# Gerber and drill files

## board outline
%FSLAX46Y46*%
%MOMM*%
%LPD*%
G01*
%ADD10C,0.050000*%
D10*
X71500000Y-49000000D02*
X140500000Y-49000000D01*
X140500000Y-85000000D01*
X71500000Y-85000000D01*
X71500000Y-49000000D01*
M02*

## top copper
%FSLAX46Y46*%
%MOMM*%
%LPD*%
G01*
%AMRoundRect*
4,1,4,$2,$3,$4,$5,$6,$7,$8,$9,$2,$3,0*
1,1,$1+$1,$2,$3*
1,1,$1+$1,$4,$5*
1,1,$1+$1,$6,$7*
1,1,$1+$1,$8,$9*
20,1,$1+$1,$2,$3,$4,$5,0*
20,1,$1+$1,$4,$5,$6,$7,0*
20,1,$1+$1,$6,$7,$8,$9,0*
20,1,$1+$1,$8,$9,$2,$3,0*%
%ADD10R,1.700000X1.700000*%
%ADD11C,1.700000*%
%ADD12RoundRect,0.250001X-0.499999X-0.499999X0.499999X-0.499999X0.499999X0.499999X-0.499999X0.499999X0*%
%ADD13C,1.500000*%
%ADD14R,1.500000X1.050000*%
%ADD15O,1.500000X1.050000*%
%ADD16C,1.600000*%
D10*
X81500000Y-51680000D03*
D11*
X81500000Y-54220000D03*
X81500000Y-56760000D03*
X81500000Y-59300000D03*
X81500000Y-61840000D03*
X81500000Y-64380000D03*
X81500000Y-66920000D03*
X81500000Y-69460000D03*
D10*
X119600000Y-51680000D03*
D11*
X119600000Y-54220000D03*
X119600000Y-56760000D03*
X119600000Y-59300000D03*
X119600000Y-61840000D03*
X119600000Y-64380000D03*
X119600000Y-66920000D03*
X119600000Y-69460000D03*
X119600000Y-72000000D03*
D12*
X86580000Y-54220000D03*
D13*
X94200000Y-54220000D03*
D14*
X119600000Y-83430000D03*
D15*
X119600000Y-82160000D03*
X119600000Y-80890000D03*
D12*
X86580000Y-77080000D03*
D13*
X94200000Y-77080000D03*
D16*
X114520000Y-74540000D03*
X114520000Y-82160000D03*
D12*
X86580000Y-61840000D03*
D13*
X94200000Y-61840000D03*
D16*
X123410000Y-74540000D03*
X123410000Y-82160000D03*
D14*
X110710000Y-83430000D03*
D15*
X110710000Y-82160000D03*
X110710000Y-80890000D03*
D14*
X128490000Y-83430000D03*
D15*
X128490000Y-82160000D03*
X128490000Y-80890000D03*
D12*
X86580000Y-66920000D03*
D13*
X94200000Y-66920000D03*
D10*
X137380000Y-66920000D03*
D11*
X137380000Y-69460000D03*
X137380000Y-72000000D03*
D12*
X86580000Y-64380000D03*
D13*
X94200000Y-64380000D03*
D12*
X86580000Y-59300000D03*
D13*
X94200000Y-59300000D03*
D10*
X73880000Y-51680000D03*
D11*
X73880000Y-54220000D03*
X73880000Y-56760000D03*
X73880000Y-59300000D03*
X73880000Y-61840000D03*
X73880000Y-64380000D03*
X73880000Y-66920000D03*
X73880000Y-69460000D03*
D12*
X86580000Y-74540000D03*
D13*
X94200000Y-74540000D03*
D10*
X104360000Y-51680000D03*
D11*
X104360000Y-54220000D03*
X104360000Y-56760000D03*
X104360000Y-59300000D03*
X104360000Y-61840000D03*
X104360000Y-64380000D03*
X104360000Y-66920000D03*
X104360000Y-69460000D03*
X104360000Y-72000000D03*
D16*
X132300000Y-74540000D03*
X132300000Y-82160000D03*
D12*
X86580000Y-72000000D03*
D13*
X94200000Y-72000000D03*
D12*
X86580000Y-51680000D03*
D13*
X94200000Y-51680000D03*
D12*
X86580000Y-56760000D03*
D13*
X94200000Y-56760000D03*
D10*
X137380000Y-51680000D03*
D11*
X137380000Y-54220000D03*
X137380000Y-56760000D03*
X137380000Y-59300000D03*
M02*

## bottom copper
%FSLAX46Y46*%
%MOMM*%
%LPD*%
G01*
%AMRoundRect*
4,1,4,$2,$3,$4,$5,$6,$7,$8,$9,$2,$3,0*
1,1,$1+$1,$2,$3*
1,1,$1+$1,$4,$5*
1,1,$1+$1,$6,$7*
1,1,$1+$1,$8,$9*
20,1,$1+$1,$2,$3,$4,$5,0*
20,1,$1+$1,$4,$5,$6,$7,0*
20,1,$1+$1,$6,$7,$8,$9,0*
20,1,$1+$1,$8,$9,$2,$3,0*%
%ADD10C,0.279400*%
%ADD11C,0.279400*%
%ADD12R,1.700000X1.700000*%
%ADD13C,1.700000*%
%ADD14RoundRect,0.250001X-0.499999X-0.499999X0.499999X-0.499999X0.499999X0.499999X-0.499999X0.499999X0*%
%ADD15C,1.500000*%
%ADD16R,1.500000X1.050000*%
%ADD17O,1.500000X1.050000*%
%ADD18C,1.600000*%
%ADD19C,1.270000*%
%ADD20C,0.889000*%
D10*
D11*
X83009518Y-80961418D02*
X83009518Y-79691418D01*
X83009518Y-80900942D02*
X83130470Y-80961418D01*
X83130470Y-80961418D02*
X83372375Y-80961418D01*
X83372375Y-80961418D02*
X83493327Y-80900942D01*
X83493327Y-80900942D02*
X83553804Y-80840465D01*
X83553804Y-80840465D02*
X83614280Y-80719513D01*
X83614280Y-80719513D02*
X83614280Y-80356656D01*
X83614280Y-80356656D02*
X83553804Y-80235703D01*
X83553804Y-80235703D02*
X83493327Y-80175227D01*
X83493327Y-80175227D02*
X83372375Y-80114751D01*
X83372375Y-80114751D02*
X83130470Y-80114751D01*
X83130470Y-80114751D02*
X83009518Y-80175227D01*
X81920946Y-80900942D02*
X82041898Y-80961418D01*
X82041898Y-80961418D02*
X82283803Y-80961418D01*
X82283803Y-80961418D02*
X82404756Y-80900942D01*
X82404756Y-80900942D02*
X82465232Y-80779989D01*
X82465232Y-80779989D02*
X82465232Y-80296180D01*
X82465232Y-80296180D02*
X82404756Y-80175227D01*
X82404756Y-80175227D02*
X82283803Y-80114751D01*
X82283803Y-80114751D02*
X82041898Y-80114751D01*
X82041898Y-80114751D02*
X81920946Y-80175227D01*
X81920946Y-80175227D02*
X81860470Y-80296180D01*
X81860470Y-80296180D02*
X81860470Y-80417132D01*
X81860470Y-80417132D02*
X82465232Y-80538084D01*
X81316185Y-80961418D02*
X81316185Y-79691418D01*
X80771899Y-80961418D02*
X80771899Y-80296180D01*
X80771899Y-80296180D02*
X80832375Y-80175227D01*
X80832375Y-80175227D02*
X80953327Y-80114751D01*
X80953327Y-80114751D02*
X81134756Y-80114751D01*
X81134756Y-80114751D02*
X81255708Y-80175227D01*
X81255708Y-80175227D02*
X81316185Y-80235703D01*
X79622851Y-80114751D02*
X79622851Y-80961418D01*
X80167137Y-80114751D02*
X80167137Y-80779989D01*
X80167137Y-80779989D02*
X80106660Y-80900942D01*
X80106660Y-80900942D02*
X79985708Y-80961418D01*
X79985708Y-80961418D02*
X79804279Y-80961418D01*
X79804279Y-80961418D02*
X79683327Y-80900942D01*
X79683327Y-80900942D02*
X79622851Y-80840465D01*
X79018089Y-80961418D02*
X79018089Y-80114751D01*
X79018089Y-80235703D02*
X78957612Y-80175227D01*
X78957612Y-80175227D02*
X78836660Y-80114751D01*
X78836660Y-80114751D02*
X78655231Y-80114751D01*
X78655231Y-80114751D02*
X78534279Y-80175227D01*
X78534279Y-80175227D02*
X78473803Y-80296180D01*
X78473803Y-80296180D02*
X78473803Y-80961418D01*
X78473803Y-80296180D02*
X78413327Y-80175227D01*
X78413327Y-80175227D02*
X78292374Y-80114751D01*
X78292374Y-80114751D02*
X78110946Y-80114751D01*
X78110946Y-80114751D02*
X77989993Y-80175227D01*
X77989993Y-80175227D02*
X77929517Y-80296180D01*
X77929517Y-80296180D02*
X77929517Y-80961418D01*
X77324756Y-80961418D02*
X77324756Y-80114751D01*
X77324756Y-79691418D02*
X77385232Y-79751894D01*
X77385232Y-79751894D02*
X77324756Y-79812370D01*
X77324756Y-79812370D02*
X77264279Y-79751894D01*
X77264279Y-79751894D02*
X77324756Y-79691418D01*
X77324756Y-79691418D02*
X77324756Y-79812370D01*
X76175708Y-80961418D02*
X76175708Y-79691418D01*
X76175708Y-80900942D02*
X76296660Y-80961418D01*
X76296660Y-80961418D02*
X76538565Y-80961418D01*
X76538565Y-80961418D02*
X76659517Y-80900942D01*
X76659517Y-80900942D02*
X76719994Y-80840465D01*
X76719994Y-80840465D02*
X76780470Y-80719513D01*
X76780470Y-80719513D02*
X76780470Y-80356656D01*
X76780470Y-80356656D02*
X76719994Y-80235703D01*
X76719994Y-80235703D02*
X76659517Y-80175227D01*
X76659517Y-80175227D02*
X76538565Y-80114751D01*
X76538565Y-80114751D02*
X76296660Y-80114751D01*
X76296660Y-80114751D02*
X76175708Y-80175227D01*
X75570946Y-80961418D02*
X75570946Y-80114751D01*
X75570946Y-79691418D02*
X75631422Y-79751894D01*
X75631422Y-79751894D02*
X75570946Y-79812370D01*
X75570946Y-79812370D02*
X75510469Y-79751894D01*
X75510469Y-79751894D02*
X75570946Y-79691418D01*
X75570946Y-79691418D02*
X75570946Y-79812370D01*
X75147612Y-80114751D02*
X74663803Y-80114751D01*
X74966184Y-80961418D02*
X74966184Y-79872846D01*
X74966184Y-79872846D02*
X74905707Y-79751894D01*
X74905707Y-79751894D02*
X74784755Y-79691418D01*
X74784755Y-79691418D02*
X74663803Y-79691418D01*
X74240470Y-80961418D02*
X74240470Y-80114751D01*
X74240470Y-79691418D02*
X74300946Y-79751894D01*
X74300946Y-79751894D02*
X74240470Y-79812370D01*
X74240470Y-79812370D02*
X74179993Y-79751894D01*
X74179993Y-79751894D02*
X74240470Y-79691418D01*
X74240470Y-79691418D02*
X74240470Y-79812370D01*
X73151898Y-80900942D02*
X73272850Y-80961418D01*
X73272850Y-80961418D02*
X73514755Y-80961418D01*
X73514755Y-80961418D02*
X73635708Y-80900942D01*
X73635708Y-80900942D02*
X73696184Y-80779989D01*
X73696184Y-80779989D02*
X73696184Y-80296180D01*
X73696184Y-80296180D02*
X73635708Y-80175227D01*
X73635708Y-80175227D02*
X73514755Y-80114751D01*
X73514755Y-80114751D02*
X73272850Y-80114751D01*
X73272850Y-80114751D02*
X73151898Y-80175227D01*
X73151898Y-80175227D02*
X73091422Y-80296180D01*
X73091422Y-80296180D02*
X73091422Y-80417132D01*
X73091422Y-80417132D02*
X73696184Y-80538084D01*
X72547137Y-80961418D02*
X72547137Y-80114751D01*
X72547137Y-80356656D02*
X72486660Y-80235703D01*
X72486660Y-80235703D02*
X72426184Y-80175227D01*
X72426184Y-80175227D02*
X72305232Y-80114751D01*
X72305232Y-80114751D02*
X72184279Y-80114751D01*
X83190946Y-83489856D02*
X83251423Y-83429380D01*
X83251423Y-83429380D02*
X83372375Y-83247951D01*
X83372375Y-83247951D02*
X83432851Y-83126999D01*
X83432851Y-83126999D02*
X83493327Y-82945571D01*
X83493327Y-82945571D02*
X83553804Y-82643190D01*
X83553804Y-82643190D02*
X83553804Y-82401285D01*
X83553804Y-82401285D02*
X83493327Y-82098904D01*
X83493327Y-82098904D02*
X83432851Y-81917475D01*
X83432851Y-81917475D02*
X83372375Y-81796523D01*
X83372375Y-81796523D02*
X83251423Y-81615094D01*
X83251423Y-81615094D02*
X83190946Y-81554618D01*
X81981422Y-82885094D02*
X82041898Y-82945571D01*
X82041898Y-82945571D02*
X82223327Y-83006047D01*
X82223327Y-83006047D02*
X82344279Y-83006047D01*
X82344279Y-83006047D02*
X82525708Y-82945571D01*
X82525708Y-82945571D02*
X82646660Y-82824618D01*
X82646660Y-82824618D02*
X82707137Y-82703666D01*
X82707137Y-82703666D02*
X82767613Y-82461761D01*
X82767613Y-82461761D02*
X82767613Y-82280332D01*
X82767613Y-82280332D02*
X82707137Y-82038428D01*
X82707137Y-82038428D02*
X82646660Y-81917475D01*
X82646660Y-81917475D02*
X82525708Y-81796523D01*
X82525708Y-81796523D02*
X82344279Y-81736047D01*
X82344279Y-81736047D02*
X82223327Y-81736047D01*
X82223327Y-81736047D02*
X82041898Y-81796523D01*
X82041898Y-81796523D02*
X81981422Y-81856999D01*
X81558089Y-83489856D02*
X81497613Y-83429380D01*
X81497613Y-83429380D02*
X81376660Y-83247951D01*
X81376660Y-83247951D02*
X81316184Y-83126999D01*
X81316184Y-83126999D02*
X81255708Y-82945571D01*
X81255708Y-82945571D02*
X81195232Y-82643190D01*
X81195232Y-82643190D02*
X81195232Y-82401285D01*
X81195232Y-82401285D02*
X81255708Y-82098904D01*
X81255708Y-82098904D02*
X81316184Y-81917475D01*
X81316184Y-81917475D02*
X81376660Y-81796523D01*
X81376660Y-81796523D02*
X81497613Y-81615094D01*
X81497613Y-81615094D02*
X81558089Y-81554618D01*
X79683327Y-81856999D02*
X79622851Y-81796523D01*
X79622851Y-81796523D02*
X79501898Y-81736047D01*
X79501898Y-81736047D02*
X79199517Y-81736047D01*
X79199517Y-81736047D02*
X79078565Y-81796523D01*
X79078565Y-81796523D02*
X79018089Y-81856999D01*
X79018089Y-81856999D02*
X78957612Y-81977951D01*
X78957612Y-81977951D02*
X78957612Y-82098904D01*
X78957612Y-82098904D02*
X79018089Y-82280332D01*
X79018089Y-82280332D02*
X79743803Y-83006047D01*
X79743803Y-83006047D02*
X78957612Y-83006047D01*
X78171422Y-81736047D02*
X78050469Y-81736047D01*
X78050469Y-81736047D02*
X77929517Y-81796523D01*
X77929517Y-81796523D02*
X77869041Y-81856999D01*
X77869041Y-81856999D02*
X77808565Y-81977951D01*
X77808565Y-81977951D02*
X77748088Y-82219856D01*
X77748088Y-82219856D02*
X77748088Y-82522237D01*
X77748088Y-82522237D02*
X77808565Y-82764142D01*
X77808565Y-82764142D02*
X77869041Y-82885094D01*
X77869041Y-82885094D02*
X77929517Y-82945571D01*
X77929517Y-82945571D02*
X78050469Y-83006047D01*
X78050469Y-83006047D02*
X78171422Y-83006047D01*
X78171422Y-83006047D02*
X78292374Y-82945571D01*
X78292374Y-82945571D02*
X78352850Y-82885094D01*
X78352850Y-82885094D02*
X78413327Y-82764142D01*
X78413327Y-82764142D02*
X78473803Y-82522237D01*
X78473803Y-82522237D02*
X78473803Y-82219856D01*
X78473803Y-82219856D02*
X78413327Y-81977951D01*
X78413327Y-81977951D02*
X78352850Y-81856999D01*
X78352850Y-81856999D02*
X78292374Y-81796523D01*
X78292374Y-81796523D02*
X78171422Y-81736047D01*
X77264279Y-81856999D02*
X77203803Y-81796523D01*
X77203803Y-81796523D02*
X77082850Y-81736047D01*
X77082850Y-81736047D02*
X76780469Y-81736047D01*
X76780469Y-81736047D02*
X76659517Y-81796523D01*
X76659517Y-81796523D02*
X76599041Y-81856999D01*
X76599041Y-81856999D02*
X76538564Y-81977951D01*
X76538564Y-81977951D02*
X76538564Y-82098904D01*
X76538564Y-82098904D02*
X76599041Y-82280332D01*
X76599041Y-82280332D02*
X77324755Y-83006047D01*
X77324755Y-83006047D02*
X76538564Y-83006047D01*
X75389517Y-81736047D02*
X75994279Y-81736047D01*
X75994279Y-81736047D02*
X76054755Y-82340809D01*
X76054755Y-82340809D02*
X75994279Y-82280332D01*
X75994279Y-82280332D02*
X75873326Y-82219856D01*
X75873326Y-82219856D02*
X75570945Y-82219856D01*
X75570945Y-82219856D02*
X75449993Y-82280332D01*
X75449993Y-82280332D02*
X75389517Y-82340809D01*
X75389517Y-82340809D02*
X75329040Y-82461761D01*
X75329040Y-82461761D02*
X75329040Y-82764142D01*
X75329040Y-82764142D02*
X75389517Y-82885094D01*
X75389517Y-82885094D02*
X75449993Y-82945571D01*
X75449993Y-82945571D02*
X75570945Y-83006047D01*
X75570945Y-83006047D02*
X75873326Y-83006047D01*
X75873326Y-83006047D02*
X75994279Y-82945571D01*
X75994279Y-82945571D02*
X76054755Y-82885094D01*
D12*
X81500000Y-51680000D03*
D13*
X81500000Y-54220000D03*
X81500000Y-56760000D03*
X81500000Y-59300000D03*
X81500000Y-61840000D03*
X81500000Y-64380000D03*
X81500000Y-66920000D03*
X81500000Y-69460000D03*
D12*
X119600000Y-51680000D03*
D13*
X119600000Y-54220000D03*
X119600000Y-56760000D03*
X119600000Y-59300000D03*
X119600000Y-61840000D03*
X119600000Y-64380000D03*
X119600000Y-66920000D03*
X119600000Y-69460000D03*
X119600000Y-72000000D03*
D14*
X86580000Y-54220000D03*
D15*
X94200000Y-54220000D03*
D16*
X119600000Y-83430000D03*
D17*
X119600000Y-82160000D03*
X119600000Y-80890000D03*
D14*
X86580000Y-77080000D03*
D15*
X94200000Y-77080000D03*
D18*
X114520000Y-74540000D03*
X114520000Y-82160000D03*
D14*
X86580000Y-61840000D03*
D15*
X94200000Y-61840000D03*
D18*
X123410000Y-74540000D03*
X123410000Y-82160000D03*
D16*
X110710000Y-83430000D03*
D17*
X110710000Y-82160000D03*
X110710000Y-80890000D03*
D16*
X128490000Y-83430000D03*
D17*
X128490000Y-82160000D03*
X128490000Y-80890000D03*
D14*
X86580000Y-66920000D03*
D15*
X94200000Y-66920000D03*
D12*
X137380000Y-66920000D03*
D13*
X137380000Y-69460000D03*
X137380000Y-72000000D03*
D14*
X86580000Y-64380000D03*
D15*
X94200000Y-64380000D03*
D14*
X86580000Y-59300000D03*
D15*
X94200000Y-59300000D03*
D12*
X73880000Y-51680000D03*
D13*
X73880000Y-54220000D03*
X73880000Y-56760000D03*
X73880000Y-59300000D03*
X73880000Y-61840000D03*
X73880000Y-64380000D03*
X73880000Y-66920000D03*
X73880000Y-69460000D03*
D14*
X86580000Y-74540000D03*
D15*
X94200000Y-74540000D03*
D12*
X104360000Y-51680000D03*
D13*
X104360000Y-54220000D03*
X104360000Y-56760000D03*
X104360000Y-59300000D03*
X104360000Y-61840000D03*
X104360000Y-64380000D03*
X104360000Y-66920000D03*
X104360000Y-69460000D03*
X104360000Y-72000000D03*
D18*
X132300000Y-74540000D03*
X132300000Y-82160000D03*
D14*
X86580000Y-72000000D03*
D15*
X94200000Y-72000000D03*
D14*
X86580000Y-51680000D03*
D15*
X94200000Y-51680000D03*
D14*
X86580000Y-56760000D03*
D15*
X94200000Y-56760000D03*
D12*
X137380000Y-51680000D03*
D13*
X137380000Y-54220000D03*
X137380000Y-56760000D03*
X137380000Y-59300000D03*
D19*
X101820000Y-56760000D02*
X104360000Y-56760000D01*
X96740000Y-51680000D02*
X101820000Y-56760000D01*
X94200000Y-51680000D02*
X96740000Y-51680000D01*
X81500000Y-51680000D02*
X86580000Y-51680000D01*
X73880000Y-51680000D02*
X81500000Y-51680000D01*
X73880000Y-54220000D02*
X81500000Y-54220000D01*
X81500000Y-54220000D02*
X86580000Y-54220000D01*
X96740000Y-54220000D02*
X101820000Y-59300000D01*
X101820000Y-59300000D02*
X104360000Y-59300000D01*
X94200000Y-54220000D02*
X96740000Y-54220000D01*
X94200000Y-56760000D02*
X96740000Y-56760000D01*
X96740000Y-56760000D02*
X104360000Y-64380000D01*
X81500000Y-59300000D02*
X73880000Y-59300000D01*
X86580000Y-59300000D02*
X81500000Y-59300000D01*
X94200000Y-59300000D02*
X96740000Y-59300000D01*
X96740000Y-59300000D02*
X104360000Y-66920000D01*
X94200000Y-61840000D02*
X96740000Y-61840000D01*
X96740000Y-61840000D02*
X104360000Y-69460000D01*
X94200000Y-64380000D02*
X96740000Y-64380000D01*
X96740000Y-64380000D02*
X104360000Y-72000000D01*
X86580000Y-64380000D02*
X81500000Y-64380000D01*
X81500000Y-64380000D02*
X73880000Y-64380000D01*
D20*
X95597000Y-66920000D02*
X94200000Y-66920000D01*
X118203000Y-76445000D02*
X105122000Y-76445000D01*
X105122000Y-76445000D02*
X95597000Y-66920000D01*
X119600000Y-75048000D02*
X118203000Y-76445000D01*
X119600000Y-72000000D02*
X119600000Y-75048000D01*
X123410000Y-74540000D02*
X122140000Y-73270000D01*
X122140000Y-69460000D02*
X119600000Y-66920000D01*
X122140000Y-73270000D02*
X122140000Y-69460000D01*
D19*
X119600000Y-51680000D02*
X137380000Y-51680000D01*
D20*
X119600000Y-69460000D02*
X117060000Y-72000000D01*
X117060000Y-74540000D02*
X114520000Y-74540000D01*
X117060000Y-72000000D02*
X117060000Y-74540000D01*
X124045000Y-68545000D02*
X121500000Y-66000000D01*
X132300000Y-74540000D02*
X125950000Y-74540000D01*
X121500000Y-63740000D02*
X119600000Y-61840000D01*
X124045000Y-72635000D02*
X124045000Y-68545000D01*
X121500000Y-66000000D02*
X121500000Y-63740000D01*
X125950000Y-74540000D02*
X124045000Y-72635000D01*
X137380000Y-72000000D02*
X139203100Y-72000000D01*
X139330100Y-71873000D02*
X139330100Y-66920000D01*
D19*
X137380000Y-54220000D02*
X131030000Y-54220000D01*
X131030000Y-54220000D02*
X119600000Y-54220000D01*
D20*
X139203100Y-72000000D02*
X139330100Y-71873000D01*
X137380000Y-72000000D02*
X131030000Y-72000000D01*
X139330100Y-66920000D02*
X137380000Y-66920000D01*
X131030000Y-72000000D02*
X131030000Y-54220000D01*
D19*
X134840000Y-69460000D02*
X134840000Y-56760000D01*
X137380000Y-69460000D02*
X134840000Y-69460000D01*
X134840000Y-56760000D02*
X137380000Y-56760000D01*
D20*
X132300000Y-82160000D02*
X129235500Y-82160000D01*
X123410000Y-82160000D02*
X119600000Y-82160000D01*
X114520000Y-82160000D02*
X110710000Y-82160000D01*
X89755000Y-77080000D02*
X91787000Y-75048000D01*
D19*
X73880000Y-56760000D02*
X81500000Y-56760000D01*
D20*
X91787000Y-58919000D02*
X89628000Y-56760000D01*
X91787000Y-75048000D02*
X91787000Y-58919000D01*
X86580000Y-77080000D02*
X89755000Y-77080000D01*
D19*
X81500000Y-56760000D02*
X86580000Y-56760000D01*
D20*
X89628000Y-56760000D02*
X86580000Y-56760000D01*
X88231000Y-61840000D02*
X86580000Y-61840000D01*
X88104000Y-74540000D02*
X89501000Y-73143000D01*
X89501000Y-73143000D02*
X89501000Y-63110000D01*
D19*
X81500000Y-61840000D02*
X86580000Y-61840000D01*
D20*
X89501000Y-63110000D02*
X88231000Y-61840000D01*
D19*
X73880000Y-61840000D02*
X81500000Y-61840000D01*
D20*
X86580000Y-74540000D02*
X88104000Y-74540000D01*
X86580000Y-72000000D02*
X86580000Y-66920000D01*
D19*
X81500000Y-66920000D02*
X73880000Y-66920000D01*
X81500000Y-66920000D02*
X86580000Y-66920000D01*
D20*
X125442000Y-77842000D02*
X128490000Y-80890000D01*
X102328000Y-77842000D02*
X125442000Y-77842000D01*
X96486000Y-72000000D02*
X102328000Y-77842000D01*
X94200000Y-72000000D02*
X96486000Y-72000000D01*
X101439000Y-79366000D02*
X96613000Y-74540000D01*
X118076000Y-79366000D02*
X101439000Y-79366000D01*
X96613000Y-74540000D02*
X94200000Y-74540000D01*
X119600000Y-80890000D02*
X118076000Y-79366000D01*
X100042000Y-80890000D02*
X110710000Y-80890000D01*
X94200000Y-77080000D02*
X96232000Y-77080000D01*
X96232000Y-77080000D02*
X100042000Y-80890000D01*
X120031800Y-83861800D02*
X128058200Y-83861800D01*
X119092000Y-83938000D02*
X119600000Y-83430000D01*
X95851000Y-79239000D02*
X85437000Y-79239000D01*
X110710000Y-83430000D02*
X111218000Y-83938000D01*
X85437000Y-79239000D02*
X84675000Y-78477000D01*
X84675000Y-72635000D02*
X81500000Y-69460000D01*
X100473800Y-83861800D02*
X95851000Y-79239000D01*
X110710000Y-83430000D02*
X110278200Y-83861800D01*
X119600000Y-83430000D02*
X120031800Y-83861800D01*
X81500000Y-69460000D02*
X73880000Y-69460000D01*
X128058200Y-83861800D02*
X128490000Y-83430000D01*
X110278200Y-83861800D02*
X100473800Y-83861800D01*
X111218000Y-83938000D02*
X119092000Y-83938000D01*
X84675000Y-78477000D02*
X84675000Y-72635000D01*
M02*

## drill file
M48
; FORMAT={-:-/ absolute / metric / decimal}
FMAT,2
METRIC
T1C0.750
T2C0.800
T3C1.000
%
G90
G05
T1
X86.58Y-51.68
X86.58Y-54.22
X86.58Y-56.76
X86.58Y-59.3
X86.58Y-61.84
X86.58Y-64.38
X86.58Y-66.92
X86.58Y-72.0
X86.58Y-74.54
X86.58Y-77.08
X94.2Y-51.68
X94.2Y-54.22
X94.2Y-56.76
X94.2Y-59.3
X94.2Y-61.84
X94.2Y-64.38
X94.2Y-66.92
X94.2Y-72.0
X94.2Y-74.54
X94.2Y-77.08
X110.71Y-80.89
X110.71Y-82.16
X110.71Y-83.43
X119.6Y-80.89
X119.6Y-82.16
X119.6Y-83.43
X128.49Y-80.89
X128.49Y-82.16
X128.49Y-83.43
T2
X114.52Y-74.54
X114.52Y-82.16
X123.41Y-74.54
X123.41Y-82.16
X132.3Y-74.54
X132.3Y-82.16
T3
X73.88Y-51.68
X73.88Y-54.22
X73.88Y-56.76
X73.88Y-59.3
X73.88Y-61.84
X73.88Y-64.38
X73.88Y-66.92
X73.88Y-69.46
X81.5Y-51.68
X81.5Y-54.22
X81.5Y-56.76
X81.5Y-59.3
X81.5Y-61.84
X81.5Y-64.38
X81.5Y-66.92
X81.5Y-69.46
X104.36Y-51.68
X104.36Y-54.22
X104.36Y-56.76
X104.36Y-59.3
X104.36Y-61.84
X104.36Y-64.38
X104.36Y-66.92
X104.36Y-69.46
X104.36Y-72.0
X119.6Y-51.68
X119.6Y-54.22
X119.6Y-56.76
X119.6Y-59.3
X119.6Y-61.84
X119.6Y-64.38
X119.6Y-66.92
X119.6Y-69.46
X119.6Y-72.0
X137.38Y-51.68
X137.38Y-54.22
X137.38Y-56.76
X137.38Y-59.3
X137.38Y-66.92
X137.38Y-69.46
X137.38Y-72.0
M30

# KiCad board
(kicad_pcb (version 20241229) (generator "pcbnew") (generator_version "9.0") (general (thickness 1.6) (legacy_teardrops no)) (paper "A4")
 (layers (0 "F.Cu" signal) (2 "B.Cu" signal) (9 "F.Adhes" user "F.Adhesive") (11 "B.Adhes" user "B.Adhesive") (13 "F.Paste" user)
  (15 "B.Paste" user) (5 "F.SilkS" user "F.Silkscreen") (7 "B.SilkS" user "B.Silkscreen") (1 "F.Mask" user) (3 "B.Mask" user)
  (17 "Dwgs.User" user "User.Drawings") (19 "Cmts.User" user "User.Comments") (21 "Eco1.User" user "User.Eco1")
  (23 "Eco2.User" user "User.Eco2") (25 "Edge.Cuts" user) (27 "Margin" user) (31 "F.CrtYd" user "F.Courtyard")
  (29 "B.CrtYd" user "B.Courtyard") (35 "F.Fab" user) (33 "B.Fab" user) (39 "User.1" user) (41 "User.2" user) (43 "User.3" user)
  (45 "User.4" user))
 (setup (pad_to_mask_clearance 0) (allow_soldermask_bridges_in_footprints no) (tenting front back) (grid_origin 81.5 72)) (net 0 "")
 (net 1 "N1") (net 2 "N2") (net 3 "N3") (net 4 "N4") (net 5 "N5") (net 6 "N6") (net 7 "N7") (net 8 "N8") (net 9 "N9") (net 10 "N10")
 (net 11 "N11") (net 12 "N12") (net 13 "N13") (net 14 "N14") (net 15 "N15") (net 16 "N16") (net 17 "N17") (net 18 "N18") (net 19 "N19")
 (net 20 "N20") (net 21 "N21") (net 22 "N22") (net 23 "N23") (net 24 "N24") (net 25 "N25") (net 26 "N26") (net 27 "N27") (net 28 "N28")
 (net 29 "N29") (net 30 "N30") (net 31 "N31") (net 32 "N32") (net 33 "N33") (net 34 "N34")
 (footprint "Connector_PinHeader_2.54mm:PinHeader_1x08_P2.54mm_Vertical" (layer "F.Cu") (at 81.5 51.68)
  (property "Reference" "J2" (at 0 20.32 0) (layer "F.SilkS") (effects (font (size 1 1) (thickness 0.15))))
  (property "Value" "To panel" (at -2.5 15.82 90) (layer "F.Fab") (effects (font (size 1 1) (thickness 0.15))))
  (pad "1" thru_hole rect (at 0 0) (size 1.7 1.7) (drill 1) (layers "*.Cu" "*.Mask") (remove_unused_layers no) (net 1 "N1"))
  (pad "2" thru_hole circle (at 0 2.54) (size 1.7 1.7) (drill 1) (layers "*.Cu" "*.Mask") (remove_unused_layers no) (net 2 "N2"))
  (pad "3" thru_hole circle (at 0 5.08) (size 1.7 1.7) (drill 1) (layers "*.Cu" "*.Mask") (remove_unused_layers no) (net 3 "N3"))
  (pad "4" thru_hole circle (at 0 7.62) (size 1.7 1.7) (drill 1) (layers "*.Cu" "*.Mask") (remove_unused_layers no) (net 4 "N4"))
  (pad "5" thru_hole circle (at 0 10.16) (size 1.7 1.7) (drill 1) (layers "*.Cu" "*.Mask") (remove_unused_layers no) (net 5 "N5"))
  (pad "6" thru_hole circle (at 0 12.7) (size 1.7 1.7) (drill 1) (layers "*.Cu" "*.Mask") (remove_unused_layers no) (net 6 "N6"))
  (pad "7" thru_hole circle (at 0 15.24) (size 1.7 1.7) (drill 1) (layers "*.Cu" "*.Mask") (remove_unused_layers no) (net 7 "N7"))
  (pad "8" thru_hole circle (at 0 17.78) (size 1.7 1.7) (drill 1) (layers "*.Cu" "*.Mask") (remove_unused_layers no) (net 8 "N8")))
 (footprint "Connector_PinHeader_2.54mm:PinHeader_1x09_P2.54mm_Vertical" (layer "F.Cu") (at 119.6 51.68)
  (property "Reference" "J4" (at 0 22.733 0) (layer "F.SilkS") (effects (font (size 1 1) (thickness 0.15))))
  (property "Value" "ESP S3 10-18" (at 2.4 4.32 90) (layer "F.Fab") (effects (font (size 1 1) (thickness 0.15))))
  (pad "1" thru_hole rect (at 0 0) (size 1.7 1.7) (drill 1) (layers "*.Cu" "*.Mask") (remove_unused_layers no) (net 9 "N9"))
  (pad "2" thru_hole circle (at 0 2.54) (size 1.7 1.7) (drill 1) (layers "*.Cu" "*.Mask") (remove_unused_layers no) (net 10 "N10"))
  (pad "3" thru_hole circle (at 0 5.08) (size 1.7 1.7) (drill 1) (layers "*.Cu" "*.Mask") (remove_unused_layers no) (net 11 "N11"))
  (pad "4" thru_hole circle (at 0 7.62) (size 1.7 1.7) (drill 1) (layers "*.Cu" "*.Mask") (remove_unused_layers no) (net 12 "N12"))
  (pad "5" thru_hole circle (at 0 10.16) (size 1.7 1.7) (drill 1) (layers "*.Cu" "*.Mask") (remove_unused_layers no) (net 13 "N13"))
  (pad "6" thru_hole circle (at 0 12.7) (size 1.7 1.7) (drill 1) (layers "*.Cu" "*.Mask") (remove_unused_layers no) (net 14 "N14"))
  (pad "7" thru_hole circle (at 0 15.24) (size 1.7 1.7) (drill 1) (layers "*.Cu" "*.Mask") (remove_unused_layers no) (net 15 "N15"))
  (pad "8" thru_hole circle (at 0 17.78) (size 1.7 1.7) (drill 1) (layers "*.Cu" "*.Mask") (remove_unused_layers no) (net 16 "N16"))
  (pad "9" thru_hole circle (at 0 20.32) (size 1.7 1.7) (drill 1) (layers "*.Cu" "*.Mask") (remove_unused_layers no) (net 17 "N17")))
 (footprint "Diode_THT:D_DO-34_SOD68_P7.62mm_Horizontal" (layer "F.Cu") (at 86.58 54.22)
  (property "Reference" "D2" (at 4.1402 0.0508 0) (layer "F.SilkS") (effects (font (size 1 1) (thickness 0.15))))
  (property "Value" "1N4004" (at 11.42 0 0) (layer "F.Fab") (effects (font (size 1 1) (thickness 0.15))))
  (pad "1" thru_hole roundrect (at 0 0) (size 1.5 1.5) (drill 0.75) (layers "*.Cu" "*.Mask") (remove_unused_layers no)
   (roundrect_rratio 0.166667) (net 2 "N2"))
  (pad "2" thru_hole circle (at 7.62 0) (size 1.5 1.5) (drill 0.75) (layers "*.Cu" "*.Mask") (remove_unused_layers no) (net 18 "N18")))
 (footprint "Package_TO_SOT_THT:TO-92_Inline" (layer "F.Cu") (at 119.6 83.43 90)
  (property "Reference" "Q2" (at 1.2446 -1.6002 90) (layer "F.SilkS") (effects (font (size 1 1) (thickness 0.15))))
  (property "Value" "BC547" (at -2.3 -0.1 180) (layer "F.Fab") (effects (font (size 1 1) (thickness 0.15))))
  (pad "1" thru_hole rect (at 0 0 90) (size 1.05 1.5) (drill 0.75) (layers "*.Cu" "*.Mask") (remove_unused_layers no) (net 8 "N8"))
  (pad "2" thru_hole oval (at 1.27 0 90) (size 1.05 1.5) (drill 0.75) (layers "*.Cu" "*.Mask") (remove_unused_layers no) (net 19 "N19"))
  (pad "3" thru_hole oval (at 2.54 0 90) (size 1.05 1.5) (drill 0.75) (layers "*.Cu" "*.Mask") (remove_unused_layers no) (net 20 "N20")))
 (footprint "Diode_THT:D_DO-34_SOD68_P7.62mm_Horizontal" (layer "F.Cu") (at 86.58 77.08)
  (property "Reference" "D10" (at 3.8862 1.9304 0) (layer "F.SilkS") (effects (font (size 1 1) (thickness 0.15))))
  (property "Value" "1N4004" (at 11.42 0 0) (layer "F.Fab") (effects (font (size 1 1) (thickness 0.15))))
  (pad "1" thru_hole roundrect (at 0 0) (size 1.5 1.5) (drill 0.75) (layers "*.Cu" "*.Mask") (remove_unused_layers no)
   (roundrect_rratio 0.166667) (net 3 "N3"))
  (pad "2" thru_hole circle (at 7.62 0) (size 1.5 1.5) (drill 0.75) (layers "*.Cu" "*.Mask") (remove_unused_layers no) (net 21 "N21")))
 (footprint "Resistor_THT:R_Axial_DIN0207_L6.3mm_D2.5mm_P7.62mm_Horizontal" (layer "F.Cu") (at 114.52 74.54 -90)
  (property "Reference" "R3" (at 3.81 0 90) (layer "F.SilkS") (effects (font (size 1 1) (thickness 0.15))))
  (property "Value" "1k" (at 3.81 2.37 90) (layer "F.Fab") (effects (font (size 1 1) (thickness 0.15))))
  (pad "1" thru_hole circle (at 0 0 270) (size 1.6 1.6) (drill 0.8) (layers "*.Cu" "*.Mask") (remove_unused_layers no) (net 16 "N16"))
  (pad "2" thru_hole circle (at 7.62 0 270) (size 1.6 1.6) (drill 0.8) (layers "*.Cu" "*.Mask") (remove_unused_layers no) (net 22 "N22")))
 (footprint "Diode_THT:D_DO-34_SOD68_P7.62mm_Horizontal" (layer "F.Cu") (at 86.58 61.84)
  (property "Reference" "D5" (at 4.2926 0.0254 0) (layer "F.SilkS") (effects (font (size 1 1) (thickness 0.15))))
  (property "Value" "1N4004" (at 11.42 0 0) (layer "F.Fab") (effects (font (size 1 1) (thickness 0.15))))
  (pad "1" thru_hole roundrect (at 0 0) (size 1.5 1.5) (drill 0.75) (layers "*.Cu" "*.Mask") (remove_unused_layers no)
   (roundrect_rratio 0.166667) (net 5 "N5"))
  (pad "2" thru_hole circle (at 7.62 0) (size 1.5 1.5) (drill 0.75) (layers "*.Cu" "*.Mask") (remove_unused_layers no) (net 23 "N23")))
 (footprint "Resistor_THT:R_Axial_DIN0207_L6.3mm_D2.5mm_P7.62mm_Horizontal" (layer "F.Cu") (at 123.41 74.54 -90)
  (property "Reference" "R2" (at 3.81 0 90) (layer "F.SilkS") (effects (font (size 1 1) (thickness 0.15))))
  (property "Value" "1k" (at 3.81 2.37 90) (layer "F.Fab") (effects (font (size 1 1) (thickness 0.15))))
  (pad "1" thru_hole circle (at 0 0 270) (size 1.6 1.6) (drill 0.8) (layers "*.Cu" "*.Mask") (remove_unused_layers no) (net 15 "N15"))
  (pad "2" thru_hole circle (at 7.62 0 270) (size 1.6 1.6) (drill 0.8) (layers "*.Cu" "*.Mask") (remove_unused_layers no) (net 19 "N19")))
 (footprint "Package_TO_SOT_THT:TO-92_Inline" (layer "F.Cu") (at 110.71 83.43 90)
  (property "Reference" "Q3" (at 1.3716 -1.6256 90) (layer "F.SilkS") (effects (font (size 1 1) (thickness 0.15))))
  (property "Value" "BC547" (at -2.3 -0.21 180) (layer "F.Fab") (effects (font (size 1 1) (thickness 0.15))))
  (pad "1" thru_hole rect (at 0 0 90) (size 1.05 1.5) (drill 0.75) (layers "*.Cu" "*.Mask") (remove_unused_layers no) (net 8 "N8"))
  (pad "2" thru_hole oval (at 1.27 0 90) (size 1.05 1.5) (drill 0.75) (layers "*.Cu" "*.Mask") (remove_unused_layers no) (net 22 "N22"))
  (pad "3" thru_hole oval (at 2.54 0 90) (size 1.05 1.5) (drill 0.75) (layers "*.Cu" "*.Mask") (remove_unused_layers no) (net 21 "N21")))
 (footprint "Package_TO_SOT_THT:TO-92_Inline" (layer "F.Cu") (at 128.49 83.43 90)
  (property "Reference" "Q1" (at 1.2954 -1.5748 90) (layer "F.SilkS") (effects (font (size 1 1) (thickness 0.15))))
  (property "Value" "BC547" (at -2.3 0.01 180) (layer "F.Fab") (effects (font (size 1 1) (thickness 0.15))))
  (pad "1" thru_hole rect (at 0 0 90) (size 1.05 1.5) (drill 0.75) (layers "*.Cu" "*.Mask") (remove_unused_layers no) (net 8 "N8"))
  (pad "2" thru_hole oval (at 1.27 0 90) (size 1.05 1.5) (drill 0.75) (layers "*.Cu" "*.Mask") (remove_unused_layers no) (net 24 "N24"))
  (pad "3" thru_hole oval (at 2.54 0 90) (size 1.05 1.5) (drill 0.75) (layers "*.Cu" "*.Mask") (remove_unused_layers no) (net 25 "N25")))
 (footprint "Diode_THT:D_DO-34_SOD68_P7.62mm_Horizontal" (layer "F.Cu") (at 86.58 66.92)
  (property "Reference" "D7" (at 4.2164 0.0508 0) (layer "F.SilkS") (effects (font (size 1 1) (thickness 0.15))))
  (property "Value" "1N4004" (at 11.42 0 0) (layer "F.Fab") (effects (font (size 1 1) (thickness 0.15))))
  (pad "1" thru_hole roundrect (at 0 0) (size 1.5 1.5) (drill 0.75) (layers "*.Cu" "*.Mask") (remove_unused_layers no)
   (roundrect_rratio 0.166667) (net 7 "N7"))
  (pad "2" thru_hole circle (at 7.62 0) (size 1.5 1.5) (drill 0.75) (layers "*.Cu" "*.Mask") (remove_unused_layers no) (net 17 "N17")))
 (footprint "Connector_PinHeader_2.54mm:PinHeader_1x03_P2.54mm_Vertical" (layer "F.Cu") (at 137.38 66.92)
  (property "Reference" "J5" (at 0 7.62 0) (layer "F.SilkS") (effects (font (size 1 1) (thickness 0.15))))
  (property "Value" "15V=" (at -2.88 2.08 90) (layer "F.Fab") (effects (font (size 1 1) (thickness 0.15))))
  (pad "1" thru_hole rect (at 0 0) (size 1.7 1.7) (drill 1) (layers "*.Cu" "*.Mask") (remove_unused_layers no) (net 10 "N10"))
  (pad "2" thru_hole circle (at 0 2.54) (size 1.7 1.7) (drill 1) (layers "*.Cu" "*.Mask") (remove_unused_layers no) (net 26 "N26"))
  (pad "3" thru_hole circle (at 0 5.08) (size 1.7 1.7) (drill 1) (layers "*.Cu" "*.Mask") (remove_unused_layers no) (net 10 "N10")))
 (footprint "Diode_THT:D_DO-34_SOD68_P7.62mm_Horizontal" (layer "F.Cu") (at 86.58 64.38)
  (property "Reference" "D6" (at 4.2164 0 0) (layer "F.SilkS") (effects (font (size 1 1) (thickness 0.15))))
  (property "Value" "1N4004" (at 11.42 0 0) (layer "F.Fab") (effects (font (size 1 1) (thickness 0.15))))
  (pad "1" thru_hole roundrect (at 0 0) (size 1.5 1.5) (drill 0.75) (layers "*.Cu" "*.Mask") (remove_unused_layers no)
   (roundrect_rratio 0.166667) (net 6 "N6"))
  (pad "2" thru_hole circle (at 7.62 0) (size 1.5 1.5) (drill 0.75) (layers "*.Cu" "*.Mask") (remove_unused_layers no) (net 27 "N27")))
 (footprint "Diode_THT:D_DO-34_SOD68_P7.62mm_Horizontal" (layer "F.Cu") (at 86.58 59.3)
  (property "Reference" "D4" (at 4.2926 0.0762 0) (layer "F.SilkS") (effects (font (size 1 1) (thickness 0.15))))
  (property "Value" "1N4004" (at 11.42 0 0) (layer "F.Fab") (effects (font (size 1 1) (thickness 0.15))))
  (pad "1" thru_hole roundrect (at 0 0) (size 1.5 1.5) (drill 0.75) (layers "*.Cu" "*.Mask") (remove_unused_layers no)
   (roundrect_rratio 0.166667) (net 4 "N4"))
  (pad "2" thru_hole circle (at 7.62 0) (size 1.5 1.5) (drill 0.75) (layers "*.Cu" "*.Mask") (remove_unused_layers no) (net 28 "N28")))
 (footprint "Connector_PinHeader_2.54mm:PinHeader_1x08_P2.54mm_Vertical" (layer "F.Cu") (at 73.88 51.68)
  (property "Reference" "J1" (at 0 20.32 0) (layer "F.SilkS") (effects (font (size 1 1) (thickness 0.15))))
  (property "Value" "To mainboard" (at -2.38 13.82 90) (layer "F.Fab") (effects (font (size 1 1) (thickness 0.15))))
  (pad "1" thru_hole rect (at 0 0) (size 1.7 1.7) (drill 1) (layers "*.Cu" "*.Mask") (remove_unused_layers no) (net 1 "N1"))
  (pad "2" thru_hole circle (at 0 2.54) (size 1.7 1.7) (drill 1) (layers "*.Cu" "*.Mask") (remove_unused_layers no) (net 2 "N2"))
  (pad "3" thru_hole circle (at 0 5.08) (size 1.7 1.7) (drill 1) (layers "*.Cu" "*.Mask") (remove_unused_layers no) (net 3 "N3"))
  (pad "4" thru_hole circle (at 0 7.62) (size 1.7 1.7) (drill 1) (layers "*.Cu" "*.Mask") (remove_unused_layers no) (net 4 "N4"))
  (pad "5" thru_hole circle (at 0 10.16) (size 1.7 1.7) (drill 1) (layers "*.Cu" "*.Mask") (remove_unused_layers no) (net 5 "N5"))
  (pad "6" thru_hole circle (at 0 12.7) (size 1.7 1.7) (drill 1) (layers "*.Cu" "*.Mask") (remove_unused_layers no) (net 6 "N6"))
  (pad "7" thru_hole circle (at 0 15.24) (size 1.7 1.7) (drill 1) (layers "*.Cu" "*.Mask") (remove_unused_layers no) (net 7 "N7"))
  (pad "8" thru_hole circle (at 0 17.78) (size 1.7 1.7) (drill 1) (layers "*.Cu" "*.Mask") (remove_unused_layers no) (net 8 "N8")))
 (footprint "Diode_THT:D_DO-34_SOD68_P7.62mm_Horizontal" (layer "F.Cu") (at 86.58 74.54)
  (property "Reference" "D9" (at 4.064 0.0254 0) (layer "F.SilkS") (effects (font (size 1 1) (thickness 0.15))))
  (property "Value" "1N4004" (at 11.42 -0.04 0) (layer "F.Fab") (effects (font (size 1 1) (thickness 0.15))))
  (pad "1" thru_hole roundrect (at 0 0) (size 1.5 1.5) (drill 0.75) (layers "*.Cu" "*.Mask") (remove_unused_layers no)
   (roundrect_rratio 0.166667) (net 5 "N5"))
  (pad "2" thru_hole circle (at 7.62 0) (size 1.5 1.5) (drill 0.75) (layers "*.Cu" "*.Mask") (remove_unused_layers no) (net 20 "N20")))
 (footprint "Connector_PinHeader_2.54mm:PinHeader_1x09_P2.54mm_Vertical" (layer "F.Cu") (at 104.36 51.68)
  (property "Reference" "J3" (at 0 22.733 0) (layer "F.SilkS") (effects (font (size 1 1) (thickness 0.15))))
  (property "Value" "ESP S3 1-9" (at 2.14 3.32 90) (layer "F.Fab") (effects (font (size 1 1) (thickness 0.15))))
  (pad "1" thru_hole rect (at 0 0) (size 1.7 1.7) (drill 1) (layers "*.Cu" "*.Mask") (remove_unused_layers no) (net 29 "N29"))
  (pad "2" thru_hole circle (at 0 2.54) (size 1.7 1.7) (drill 1) (layers "*.Cu" "*.Mask") (remove_unused_layers no) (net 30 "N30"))
  (pad "3" thru_hole circle (at 0 5.08) (size 1.7 1.7) (drill 1) (layers "*.Cu" "*.Mask") (remove_unused_layers no) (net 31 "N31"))
  (pad "4" thru_hole circle (at 0 7.62) (size 1.7 1.7) (drill 1) (layers "*.Cu" "*.Mask") (remove_unused_layers no) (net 18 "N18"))
  (pad "5" thru_hole circle (at 0 10.16) (size 1.7 1.7) (drill 1) (layers "*.Cu" "*.Mask") (remove_unused_layers no) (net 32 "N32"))
  (pad "6" thru_hole circle (at 0 12.7) (size 1.7 1.7) (drill 1) (layers "*.Cu" "*.Mask") (remove_unused_layers no) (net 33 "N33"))
  (pad "7" thru_hole circle (at 0 15.24) (size 1.7 1.7) (drill 1) (layers "*.Cu" "*.Mask") (remove_unused_layers no) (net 28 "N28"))
  (pad "8" thru_hole circle (at 0 17.78) (size 1.7 1.7) (drill 1) (layers "*.Cu" "*.Mask") (remove_unused_layers no) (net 23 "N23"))
  (pad "9" thru_hole circle (at 0 20.32) (size 1.7 1.7) (drill 1) (layers "*.Cu" "*.Mask") (remove_unused_layers no) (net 27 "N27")))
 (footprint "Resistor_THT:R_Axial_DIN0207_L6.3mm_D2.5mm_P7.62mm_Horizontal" (layer "F.Cu") (at 132.3 74.54 -90)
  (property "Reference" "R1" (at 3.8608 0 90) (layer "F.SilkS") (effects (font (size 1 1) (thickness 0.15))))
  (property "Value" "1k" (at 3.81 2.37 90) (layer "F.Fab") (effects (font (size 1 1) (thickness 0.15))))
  (pad "1" thru_hole circle (at 0 0 270) (size 1.6 1.6) (drill 0.8) (layers "*.Cu" "*.Mask") (remove_unused_layers no) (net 13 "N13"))
  (pad "2" thru_hole circle (at 7.62 0 270) (size 1.6 1.6) (drill 0.8) (layers "*.Cu" "*.Mask") (remove_unused_layers no) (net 24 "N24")))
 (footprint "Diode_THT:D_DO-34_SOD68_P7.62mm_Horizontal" (layer "F.Cu") (at 86.58 72)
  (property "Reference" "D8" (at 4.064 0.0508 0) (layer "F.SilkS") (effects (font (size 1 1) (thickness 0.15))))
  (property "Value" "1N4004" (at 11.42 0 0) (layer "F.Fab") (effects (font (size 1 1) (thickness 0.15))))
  (pad "1" thru_hole roundrect (at 0 0) (size 1.5 1.5) (drill 0.75) (layers "*.Cu" "*.Mask") (remove_unused_layers no)
   (roundrect_rratio 0.166667) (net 7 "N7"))
  (pad "2" thru_hole circle (at 7.62 0) (size 1.5 1.5) (drill 0.75) (layers "*.Cu" "*.Mask") (remove_unused_layers no) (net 25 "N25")))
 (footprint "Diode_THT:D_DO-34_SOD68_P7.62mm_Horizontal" (layer "F.Cu") (at 86.58 51.68)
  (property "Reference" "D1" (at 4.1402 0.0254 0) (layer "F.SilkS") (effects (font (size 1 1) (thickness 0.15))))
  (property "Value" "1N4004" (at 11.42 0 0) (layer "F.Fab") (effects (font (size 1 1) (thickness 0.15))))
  (pad "1" thru_hole roundrect (at 0 0) (size 1.5 1.5) (drill 0.75) (layers "*.Cu" "*.Mask") (remove_unused_layers no)
   (roundrect_rratio 0.166667) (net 1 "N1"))
  (pad "2" thru_hole circle (at 7.62 0) (size 1.5 1.5) (drill 0.75) (layers "*.Cu" "*.Mask") (remove_unused_layers no) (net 31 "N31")))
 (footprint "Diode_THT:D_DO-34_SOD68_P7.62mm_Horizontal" (layer "F.Cu") (at 86.58 56.76)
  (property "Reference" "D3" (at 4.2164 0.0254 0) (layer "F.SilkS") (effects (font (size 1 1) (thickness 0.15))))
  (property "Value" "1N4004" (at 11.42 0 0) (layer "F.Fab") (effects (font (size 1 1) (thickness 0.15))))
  (pad "1" thru_hole roundrect (at 0 0) (size 1.5 1.5) (drill 0.75) (layers "*.Cu" "*.Mask") (remove_unused_layers no)
   (roundrect_rratio 0.166667) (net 3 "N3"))
  (pad "2" thru_hole circle (at 7.62 0) (size 1.5 1.5) (drill 0.75) (layers "*.Cu" "*.Mask") (remove_unused_layers no) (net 33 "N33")))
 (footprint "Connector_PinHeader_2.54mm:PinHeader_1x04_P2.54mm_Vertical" (layer "F.Cu") (at 137.38 51.68)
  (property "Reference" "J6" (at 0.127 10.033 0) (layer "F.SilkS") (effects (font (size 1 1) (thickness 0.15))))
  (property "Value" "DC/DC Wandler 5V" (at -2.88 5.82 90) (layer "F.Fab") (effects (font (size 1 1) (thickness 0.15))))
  (pad "1" thru_hole rect (at 0 0) (size 1.7 1.7) (drill 1) (layers "*.Cu" "*.Mask") (remove_unused_layers no) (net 9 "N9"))
  (pad "2" thru_hole circle (at 0 2.54) (size 1.7 1.7) (drill 1) (layers "*.Cu" "*.Mask") (remove_unused_layers no) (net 10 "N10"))
  (pad "3" thru_hole circle (at 0 5.08) (size 1.7 1.7) (drill 1) (layers "*.Cu" "*.Mask") (remove_unused_layers no) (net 26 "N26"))
  (pad "4" thru_hole circle (at 0 7.62) (size 1.7 1.7) (drill 1) (layers "*.Cu" "*.Mask") (remove_unused_layers no) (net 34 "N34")))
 (gr_rect (start 71.5 49) (end 140.5 85) (stroke (width 0.05) (type default)) (fill no) (layer "Edge.Cuts"))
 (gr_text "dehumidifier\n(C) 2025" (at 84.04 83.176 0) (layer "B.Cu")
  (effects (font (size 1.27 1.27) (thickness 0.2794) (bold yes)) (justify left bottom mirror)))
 (segment (start 101.82 56.76) (end 104.36 56.76) (width 1.27) (layer "B.Cu") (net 31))
 (segment (start 96.74 51.68) (end 101.82 56.76) (width 1.27) (layer "B.Cu") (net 31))
 (segment (start 94.2 51.68) (end 96.74 51.68) (width 1.27) (layer "B.Cu") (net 31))
 (segment (start 81.5 51.68) (end 86.58 51.68) (width 1.27) (layer "B.Cu") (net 1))
 (segment (start 73.88 51.68) (end 81.5 51.68) (width 1.27) (layer "B.Cu") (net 1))
 (segment (start 73.88 54.22) (end 81.5 54.22) (width 1.27) (layer "B.Cu") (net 2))
 (segment (start 81.5 54.22) (end 86.58 54.22) (width 1.27) (layer "B.Cu") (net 2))
 (segment (start 96.74 54.22) (end 101.82 59.3) (width 1.27) (layer "B.Cu") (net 18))
 (segment (start 101.82 59.3) (end 104.36 59.3) (width 1.27) (layer "B.Cu") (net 18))
 (segment (start 94.2 54.22) (end 96.74 54.22) (width 1.27) (layer "B.Cu") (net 18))
 (segment (start 94.2 56.76) (end 96.74 56.76) (width 1.27) (layer "B.Cu") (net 33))
 (segment (start 96.74 56.76) (end 104.36 64.38) (width 1.27) (layer "B.Cu") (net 33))
 (segment (start 81.5 59.3) (end 73.88 59.3) (width 1.27) (layer "B.Cu") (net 4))
 (segment (start 86.58 59.3) (end 81.5 59.3) (width 1.27) (layer "B.Cu") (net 4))
 (segment (start 94.2 59.3) (end 96.74 59.3) (width 1.27) (layer "B.Cu") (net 28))
 (segment (start 96.74 59.3) (end 104.36 66.92) (width 1.27) (layer "B.Cu") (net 28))
 (segment (start 94.2 61.84) (end 96.74 61.84) (width 1.27) (layer "B.Cu") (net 23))
 (segment (start 96.74 61.84) (end 104.36 69.46) (width 1.27) (layer "B.Cu") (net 23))
 (segment (start 94.2 64.38) (end 96.74 64.38) (width 1.27) (layer "B.Cu") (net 27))
 (segment (start 96.74 64.38) (end 104.36 72) (width 1.27) (layer "B.Cu") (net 27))
 (segment (start 86.58 64.38) (end 81.5 64.38) (width 1.27) (layer "B.Cu") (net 6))
 (segment (start 81.5 64.38) (end 73.88 64.38) (width 1.27) (layer "B.Cu") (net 6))
 (segment (start 95.597 66.92) (end 94.2 66.92) (width 0.889) (layer "B.Cu") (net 17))
 (segment (start 118.203 76.445) (end 105.122 76.445) (width 0.889) (layer "B.Cu") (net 17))
 (segment (start 105.122 76.445) (end 95.597 66.92) (width 0.889) (layer "B.Cu") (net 17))
 (segment (start 119.6 75.048) (end 118.203 76.445) (width 0.889) (layer "B.Cu") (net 17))
 (segment (start 119.6 72) (end 119.6 75.048) (width 0.889) (layer "B.Cu") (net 17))
 (segment (start 123.41 74.54) (end 122.14 73.27) (width 0.889) (layer "B.Cu") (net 15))
 (segment (start 122.14 69.46) (end 119.6 66.92) (width 0.889) (layer "B.Cu") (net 15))
 (segment (start 122.14 73.27) (end 122.14 69.46) (width 0.889) (layer "B.Cu") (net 15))
 (segment (start 119.6 51.68) (end 137.38 51.68) (width 1.27) (layer "B.Cu") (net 9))
 (segment (start 119.6 69.46) (end 117.06 72) (width 0.889) (layer "B.Cu") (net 16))
 (segment (start 117.06 74.54) (end 114.52 74.54) (width 0.889) (layer "B.Cu") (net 16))
 (segment (start 117.06 72) (end 117.06 74.54) (width 0.889) (layer "B.Cu") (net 16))
 (segment (start 124.045 68.545) (end 121.5 66) (width 0.889) (layer "B.Cu") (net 13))
 (segment (start 132.3 74.54) (end 125.95 74.54) (width 0.889) (layer "B.Cu") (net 13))
 (segment (start 121.5 63.74) (end 119.6 61.84) (width 0.889) (layer "B.Cu") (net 13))
 (segment (start 124.045 72.635) (end 124.045 68.545) (width 0.889) (layer "B.Cu") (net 13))
 (segment (start 121.5 66) (end 121.5 63.74) (width 0.889) (layer "B.Cu") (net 13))
 (segment (start 125.95 74.54) (end 124.045 72.635) (width 0.889) (layer "B.Cu") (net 13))
 (segment (start 137.38 72) (end 139.2031 72) (width 0.889) (layer "B.Cu") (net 10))
 (segment (start 139.3301 71.873) (end 139.3301 66.92) (width 0.889) (layer "B.Cu") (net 10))
 (segment (start 137.38 54.22) (end 131.03 54.22) (width 1.27) (layer "B.Cu") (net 10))
 (segment (start 131.03 54.22) (end 119.6 54.22) (width 1.27) (layer "B.Cu") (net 10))
 (segment (start 139.2031 72) (end 139.3301 71.873) (width 0.889) (layer "B.Cu") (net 10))
 (segment (start 137.38 72) (end 131.03 72) (width 0.889) (layer "B.Cu") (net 10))
 (segment (start 139.3301 66.92) (end 137.38 66.92) (width 0.889) (layer "B.Cu") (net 10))
 (segment (start 131.03 72) (end 131.03 54.22) (width 0.889) (layer "B.Cu") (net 10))
 (segment (start 134.84 69.46) (end 134.84 56.76) (width 1.27) (layer "B.Cu") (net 26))
 (segment (start 137.38 69.46) (end 134.84 69.46) (width 1.27) (layer "B.Cu") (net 26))
 (segment (start 134.84 56.76) (end 137.38 56.76) (width 1.27) (layer "B.Cu") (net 26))
 (segment (start 132.3 82.16) (end 129.2355 82.16) (width 0.889) (layer "B.Cu") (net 24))
 (segment (start 123.41 82.16) (end 119.6 82.16) (width 0.889) (layer "B.Cu") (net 19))
 (segment (start 114.52 82.16) (end 110.71 82.16) (width 0.889) (layer "B.Cu") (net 22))
 (segment (start 89.755 77.08) (end 91.787 75.048) (width 0.889) (layer "B.Cu") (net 3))
 (segment (start 73.88 56.76) (end 81.5 56.76) (width 1.27) (layer "B.Cu") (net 3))
 (segment (start 91.787 58.919) (end 89.628 56.76) (width 0.889) (layer "B.Cu") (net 3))
 (segment (start 91.787 75.048) (end 91.787 58.919) (width 0.889) (layer "B.Cu") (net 3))
 (segment (start 86.58 77.08) (end 89.755 77.08) (width 0.889) (layer "B.Cu") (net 3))
 (segment (start 81.5 56.76) (end 86.58 56.76) (width 1.27) (layer "B.Cu") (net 3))
 (segment (start 89.628 56.76) (end 86.58 56.76) (width 0.889) (layer "B.Cu") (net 3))
 (segment (start 88.231 61.84) (end 86.58 61.84) (width 0.889) (layer "B.Cu") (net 5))
 (segment (start 88.104 74.54) (end 89.501 73.143) (width 0.889) (layer "B.Cu") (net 5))
 (segment (start 89.501 73.143) (end 89.501 63.11) (width 0.889) (layer "B.Cu") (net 5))
 (segment (start 81.5 61.84) (end 86.58 61.84) (width 1.27) (layer "B.Cu") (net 5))
 (segment (start 89.501 63.11) (end 88.231 61.84) (width 0.889) (layer "B.Cu") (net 5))
 (segment (start 73.88 61.84) (end 81.5 61.84) (width 1.27) (layer "B.Cu") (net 5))
 (segment (start 86.58 74.54) (end 88.104 74.54) (width 0.889) (layer "B.Cu") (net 5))
 (segment (start 86.58 72) (end 86.58 66.92) (width 0.889) (layer "B.Cu") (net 7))
 (segment (start 81.5 66.92) (end 73.88 66.92) (width 1.27) (layer "B.Cu") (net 7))
 (segment (start 81.5 66.92) (end 86.58 66.92) (width 1.27) (layer "B.Cu") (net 7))
 (segment (start 125.442 77.842) (end 128.49 80.89) (width 0.889) (layer "B.Cu") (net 25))
 (segment (start 102.328 77.842) (end 125.442 77.842) (width 0.889) (layer "B.Cu") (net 25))
 (segment (start 96.486 72) (end 102.328 77.842) (width 0.889) (layer "B.Cu") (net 25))
 (segment (start 94.2 72) (end 96.486 72) (width 0.889) (layer "B.Cu") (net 25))
 (segment (start 101.439 79.366) (end 96.613 74.54) (width 0.889) (layer "B.Cu") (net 20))
 (segment (start 118.076 79.366) (end 101.439 79.366) (width 0.889) (layer "B.Cu") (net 20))
 (segment (start 96.613 74.54) (end 94.2 74.54) (width 0.889) (layer "B.Cu") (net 20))
 (segment (start 119.6 80.89) (end 118.076 79.366) (width 0.889) (layer "B.Cu") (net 20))
 (segment (start 100.042 80.89) (end 110.71 80.89) (width 0.889) (layer "B.Cu") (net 21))
 (segment (start 94.2 77.08) (end 96.232 77.08) (width 0.889) (layer "B.Cu") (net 21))
 (segment (start 96.232 77.08) (end 100.042 80.89) (width 0.889) (layer "B.Cu") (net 21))
 (segment (start 120.0318 83.8618) (end 128.0582 83.8618) (width 0.889) (layer "B.Cu") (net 8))
 (segment (start 119.092 83.938) (end 119.6 83.43) (width 0.889) (layer "B.Cu") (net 8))
 (segment (start 95.851 79.239) (end 85.437 79.239) (width 0.889) (layer "B.Cu") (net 8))
 (segment (start 110.71 83.43) (end 111.218 83.938) (width 0.889) (layer "B.Cu") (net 8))
 (segment (start 85.437 79.239) (end 84.675 78.477) (width 0.889) (layer "B.Cu") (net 8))
 (segment (start 84.675 72.635) (end 81.5 69.46) (width 0.889) (layer "B.Cu") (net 8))
 (segment (start 100.4738 83.8618) (end 95.851 79.239) (width 0.889) (layer "B.Cu") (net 8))
 (segment (start 110.71 83.43) (end 110.2782 83.8618) (width 0.889) (layer "B.Cu") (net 8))
 (segment (start 119.6 83.43) (end 120.0318 83.8618) (width 0.889) (layer "B.Cu") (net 8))
 (segment (start 81.5 69.46) (end 73.88 69.46) (width 0.889) (layer "B.Cu") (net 8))
 (segment (start 128.0582 83.8618) (end 128.49 83.43) (width 0.889) (layer "B.Cu") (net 8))
 (segment (start 110.2782 83.8618) (end 100.4738 83.8618) (width 0.889) (layer "B.Cu") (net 8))
 (segment (start 111.218 83.938) (end 119.092 83.938) (width 0.889) (layer "B.Cu") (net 8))
 (segment (start 84.675 78.477) (end 84.675 72.635) (width 0.889) (layer "B.Cu") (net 8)))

